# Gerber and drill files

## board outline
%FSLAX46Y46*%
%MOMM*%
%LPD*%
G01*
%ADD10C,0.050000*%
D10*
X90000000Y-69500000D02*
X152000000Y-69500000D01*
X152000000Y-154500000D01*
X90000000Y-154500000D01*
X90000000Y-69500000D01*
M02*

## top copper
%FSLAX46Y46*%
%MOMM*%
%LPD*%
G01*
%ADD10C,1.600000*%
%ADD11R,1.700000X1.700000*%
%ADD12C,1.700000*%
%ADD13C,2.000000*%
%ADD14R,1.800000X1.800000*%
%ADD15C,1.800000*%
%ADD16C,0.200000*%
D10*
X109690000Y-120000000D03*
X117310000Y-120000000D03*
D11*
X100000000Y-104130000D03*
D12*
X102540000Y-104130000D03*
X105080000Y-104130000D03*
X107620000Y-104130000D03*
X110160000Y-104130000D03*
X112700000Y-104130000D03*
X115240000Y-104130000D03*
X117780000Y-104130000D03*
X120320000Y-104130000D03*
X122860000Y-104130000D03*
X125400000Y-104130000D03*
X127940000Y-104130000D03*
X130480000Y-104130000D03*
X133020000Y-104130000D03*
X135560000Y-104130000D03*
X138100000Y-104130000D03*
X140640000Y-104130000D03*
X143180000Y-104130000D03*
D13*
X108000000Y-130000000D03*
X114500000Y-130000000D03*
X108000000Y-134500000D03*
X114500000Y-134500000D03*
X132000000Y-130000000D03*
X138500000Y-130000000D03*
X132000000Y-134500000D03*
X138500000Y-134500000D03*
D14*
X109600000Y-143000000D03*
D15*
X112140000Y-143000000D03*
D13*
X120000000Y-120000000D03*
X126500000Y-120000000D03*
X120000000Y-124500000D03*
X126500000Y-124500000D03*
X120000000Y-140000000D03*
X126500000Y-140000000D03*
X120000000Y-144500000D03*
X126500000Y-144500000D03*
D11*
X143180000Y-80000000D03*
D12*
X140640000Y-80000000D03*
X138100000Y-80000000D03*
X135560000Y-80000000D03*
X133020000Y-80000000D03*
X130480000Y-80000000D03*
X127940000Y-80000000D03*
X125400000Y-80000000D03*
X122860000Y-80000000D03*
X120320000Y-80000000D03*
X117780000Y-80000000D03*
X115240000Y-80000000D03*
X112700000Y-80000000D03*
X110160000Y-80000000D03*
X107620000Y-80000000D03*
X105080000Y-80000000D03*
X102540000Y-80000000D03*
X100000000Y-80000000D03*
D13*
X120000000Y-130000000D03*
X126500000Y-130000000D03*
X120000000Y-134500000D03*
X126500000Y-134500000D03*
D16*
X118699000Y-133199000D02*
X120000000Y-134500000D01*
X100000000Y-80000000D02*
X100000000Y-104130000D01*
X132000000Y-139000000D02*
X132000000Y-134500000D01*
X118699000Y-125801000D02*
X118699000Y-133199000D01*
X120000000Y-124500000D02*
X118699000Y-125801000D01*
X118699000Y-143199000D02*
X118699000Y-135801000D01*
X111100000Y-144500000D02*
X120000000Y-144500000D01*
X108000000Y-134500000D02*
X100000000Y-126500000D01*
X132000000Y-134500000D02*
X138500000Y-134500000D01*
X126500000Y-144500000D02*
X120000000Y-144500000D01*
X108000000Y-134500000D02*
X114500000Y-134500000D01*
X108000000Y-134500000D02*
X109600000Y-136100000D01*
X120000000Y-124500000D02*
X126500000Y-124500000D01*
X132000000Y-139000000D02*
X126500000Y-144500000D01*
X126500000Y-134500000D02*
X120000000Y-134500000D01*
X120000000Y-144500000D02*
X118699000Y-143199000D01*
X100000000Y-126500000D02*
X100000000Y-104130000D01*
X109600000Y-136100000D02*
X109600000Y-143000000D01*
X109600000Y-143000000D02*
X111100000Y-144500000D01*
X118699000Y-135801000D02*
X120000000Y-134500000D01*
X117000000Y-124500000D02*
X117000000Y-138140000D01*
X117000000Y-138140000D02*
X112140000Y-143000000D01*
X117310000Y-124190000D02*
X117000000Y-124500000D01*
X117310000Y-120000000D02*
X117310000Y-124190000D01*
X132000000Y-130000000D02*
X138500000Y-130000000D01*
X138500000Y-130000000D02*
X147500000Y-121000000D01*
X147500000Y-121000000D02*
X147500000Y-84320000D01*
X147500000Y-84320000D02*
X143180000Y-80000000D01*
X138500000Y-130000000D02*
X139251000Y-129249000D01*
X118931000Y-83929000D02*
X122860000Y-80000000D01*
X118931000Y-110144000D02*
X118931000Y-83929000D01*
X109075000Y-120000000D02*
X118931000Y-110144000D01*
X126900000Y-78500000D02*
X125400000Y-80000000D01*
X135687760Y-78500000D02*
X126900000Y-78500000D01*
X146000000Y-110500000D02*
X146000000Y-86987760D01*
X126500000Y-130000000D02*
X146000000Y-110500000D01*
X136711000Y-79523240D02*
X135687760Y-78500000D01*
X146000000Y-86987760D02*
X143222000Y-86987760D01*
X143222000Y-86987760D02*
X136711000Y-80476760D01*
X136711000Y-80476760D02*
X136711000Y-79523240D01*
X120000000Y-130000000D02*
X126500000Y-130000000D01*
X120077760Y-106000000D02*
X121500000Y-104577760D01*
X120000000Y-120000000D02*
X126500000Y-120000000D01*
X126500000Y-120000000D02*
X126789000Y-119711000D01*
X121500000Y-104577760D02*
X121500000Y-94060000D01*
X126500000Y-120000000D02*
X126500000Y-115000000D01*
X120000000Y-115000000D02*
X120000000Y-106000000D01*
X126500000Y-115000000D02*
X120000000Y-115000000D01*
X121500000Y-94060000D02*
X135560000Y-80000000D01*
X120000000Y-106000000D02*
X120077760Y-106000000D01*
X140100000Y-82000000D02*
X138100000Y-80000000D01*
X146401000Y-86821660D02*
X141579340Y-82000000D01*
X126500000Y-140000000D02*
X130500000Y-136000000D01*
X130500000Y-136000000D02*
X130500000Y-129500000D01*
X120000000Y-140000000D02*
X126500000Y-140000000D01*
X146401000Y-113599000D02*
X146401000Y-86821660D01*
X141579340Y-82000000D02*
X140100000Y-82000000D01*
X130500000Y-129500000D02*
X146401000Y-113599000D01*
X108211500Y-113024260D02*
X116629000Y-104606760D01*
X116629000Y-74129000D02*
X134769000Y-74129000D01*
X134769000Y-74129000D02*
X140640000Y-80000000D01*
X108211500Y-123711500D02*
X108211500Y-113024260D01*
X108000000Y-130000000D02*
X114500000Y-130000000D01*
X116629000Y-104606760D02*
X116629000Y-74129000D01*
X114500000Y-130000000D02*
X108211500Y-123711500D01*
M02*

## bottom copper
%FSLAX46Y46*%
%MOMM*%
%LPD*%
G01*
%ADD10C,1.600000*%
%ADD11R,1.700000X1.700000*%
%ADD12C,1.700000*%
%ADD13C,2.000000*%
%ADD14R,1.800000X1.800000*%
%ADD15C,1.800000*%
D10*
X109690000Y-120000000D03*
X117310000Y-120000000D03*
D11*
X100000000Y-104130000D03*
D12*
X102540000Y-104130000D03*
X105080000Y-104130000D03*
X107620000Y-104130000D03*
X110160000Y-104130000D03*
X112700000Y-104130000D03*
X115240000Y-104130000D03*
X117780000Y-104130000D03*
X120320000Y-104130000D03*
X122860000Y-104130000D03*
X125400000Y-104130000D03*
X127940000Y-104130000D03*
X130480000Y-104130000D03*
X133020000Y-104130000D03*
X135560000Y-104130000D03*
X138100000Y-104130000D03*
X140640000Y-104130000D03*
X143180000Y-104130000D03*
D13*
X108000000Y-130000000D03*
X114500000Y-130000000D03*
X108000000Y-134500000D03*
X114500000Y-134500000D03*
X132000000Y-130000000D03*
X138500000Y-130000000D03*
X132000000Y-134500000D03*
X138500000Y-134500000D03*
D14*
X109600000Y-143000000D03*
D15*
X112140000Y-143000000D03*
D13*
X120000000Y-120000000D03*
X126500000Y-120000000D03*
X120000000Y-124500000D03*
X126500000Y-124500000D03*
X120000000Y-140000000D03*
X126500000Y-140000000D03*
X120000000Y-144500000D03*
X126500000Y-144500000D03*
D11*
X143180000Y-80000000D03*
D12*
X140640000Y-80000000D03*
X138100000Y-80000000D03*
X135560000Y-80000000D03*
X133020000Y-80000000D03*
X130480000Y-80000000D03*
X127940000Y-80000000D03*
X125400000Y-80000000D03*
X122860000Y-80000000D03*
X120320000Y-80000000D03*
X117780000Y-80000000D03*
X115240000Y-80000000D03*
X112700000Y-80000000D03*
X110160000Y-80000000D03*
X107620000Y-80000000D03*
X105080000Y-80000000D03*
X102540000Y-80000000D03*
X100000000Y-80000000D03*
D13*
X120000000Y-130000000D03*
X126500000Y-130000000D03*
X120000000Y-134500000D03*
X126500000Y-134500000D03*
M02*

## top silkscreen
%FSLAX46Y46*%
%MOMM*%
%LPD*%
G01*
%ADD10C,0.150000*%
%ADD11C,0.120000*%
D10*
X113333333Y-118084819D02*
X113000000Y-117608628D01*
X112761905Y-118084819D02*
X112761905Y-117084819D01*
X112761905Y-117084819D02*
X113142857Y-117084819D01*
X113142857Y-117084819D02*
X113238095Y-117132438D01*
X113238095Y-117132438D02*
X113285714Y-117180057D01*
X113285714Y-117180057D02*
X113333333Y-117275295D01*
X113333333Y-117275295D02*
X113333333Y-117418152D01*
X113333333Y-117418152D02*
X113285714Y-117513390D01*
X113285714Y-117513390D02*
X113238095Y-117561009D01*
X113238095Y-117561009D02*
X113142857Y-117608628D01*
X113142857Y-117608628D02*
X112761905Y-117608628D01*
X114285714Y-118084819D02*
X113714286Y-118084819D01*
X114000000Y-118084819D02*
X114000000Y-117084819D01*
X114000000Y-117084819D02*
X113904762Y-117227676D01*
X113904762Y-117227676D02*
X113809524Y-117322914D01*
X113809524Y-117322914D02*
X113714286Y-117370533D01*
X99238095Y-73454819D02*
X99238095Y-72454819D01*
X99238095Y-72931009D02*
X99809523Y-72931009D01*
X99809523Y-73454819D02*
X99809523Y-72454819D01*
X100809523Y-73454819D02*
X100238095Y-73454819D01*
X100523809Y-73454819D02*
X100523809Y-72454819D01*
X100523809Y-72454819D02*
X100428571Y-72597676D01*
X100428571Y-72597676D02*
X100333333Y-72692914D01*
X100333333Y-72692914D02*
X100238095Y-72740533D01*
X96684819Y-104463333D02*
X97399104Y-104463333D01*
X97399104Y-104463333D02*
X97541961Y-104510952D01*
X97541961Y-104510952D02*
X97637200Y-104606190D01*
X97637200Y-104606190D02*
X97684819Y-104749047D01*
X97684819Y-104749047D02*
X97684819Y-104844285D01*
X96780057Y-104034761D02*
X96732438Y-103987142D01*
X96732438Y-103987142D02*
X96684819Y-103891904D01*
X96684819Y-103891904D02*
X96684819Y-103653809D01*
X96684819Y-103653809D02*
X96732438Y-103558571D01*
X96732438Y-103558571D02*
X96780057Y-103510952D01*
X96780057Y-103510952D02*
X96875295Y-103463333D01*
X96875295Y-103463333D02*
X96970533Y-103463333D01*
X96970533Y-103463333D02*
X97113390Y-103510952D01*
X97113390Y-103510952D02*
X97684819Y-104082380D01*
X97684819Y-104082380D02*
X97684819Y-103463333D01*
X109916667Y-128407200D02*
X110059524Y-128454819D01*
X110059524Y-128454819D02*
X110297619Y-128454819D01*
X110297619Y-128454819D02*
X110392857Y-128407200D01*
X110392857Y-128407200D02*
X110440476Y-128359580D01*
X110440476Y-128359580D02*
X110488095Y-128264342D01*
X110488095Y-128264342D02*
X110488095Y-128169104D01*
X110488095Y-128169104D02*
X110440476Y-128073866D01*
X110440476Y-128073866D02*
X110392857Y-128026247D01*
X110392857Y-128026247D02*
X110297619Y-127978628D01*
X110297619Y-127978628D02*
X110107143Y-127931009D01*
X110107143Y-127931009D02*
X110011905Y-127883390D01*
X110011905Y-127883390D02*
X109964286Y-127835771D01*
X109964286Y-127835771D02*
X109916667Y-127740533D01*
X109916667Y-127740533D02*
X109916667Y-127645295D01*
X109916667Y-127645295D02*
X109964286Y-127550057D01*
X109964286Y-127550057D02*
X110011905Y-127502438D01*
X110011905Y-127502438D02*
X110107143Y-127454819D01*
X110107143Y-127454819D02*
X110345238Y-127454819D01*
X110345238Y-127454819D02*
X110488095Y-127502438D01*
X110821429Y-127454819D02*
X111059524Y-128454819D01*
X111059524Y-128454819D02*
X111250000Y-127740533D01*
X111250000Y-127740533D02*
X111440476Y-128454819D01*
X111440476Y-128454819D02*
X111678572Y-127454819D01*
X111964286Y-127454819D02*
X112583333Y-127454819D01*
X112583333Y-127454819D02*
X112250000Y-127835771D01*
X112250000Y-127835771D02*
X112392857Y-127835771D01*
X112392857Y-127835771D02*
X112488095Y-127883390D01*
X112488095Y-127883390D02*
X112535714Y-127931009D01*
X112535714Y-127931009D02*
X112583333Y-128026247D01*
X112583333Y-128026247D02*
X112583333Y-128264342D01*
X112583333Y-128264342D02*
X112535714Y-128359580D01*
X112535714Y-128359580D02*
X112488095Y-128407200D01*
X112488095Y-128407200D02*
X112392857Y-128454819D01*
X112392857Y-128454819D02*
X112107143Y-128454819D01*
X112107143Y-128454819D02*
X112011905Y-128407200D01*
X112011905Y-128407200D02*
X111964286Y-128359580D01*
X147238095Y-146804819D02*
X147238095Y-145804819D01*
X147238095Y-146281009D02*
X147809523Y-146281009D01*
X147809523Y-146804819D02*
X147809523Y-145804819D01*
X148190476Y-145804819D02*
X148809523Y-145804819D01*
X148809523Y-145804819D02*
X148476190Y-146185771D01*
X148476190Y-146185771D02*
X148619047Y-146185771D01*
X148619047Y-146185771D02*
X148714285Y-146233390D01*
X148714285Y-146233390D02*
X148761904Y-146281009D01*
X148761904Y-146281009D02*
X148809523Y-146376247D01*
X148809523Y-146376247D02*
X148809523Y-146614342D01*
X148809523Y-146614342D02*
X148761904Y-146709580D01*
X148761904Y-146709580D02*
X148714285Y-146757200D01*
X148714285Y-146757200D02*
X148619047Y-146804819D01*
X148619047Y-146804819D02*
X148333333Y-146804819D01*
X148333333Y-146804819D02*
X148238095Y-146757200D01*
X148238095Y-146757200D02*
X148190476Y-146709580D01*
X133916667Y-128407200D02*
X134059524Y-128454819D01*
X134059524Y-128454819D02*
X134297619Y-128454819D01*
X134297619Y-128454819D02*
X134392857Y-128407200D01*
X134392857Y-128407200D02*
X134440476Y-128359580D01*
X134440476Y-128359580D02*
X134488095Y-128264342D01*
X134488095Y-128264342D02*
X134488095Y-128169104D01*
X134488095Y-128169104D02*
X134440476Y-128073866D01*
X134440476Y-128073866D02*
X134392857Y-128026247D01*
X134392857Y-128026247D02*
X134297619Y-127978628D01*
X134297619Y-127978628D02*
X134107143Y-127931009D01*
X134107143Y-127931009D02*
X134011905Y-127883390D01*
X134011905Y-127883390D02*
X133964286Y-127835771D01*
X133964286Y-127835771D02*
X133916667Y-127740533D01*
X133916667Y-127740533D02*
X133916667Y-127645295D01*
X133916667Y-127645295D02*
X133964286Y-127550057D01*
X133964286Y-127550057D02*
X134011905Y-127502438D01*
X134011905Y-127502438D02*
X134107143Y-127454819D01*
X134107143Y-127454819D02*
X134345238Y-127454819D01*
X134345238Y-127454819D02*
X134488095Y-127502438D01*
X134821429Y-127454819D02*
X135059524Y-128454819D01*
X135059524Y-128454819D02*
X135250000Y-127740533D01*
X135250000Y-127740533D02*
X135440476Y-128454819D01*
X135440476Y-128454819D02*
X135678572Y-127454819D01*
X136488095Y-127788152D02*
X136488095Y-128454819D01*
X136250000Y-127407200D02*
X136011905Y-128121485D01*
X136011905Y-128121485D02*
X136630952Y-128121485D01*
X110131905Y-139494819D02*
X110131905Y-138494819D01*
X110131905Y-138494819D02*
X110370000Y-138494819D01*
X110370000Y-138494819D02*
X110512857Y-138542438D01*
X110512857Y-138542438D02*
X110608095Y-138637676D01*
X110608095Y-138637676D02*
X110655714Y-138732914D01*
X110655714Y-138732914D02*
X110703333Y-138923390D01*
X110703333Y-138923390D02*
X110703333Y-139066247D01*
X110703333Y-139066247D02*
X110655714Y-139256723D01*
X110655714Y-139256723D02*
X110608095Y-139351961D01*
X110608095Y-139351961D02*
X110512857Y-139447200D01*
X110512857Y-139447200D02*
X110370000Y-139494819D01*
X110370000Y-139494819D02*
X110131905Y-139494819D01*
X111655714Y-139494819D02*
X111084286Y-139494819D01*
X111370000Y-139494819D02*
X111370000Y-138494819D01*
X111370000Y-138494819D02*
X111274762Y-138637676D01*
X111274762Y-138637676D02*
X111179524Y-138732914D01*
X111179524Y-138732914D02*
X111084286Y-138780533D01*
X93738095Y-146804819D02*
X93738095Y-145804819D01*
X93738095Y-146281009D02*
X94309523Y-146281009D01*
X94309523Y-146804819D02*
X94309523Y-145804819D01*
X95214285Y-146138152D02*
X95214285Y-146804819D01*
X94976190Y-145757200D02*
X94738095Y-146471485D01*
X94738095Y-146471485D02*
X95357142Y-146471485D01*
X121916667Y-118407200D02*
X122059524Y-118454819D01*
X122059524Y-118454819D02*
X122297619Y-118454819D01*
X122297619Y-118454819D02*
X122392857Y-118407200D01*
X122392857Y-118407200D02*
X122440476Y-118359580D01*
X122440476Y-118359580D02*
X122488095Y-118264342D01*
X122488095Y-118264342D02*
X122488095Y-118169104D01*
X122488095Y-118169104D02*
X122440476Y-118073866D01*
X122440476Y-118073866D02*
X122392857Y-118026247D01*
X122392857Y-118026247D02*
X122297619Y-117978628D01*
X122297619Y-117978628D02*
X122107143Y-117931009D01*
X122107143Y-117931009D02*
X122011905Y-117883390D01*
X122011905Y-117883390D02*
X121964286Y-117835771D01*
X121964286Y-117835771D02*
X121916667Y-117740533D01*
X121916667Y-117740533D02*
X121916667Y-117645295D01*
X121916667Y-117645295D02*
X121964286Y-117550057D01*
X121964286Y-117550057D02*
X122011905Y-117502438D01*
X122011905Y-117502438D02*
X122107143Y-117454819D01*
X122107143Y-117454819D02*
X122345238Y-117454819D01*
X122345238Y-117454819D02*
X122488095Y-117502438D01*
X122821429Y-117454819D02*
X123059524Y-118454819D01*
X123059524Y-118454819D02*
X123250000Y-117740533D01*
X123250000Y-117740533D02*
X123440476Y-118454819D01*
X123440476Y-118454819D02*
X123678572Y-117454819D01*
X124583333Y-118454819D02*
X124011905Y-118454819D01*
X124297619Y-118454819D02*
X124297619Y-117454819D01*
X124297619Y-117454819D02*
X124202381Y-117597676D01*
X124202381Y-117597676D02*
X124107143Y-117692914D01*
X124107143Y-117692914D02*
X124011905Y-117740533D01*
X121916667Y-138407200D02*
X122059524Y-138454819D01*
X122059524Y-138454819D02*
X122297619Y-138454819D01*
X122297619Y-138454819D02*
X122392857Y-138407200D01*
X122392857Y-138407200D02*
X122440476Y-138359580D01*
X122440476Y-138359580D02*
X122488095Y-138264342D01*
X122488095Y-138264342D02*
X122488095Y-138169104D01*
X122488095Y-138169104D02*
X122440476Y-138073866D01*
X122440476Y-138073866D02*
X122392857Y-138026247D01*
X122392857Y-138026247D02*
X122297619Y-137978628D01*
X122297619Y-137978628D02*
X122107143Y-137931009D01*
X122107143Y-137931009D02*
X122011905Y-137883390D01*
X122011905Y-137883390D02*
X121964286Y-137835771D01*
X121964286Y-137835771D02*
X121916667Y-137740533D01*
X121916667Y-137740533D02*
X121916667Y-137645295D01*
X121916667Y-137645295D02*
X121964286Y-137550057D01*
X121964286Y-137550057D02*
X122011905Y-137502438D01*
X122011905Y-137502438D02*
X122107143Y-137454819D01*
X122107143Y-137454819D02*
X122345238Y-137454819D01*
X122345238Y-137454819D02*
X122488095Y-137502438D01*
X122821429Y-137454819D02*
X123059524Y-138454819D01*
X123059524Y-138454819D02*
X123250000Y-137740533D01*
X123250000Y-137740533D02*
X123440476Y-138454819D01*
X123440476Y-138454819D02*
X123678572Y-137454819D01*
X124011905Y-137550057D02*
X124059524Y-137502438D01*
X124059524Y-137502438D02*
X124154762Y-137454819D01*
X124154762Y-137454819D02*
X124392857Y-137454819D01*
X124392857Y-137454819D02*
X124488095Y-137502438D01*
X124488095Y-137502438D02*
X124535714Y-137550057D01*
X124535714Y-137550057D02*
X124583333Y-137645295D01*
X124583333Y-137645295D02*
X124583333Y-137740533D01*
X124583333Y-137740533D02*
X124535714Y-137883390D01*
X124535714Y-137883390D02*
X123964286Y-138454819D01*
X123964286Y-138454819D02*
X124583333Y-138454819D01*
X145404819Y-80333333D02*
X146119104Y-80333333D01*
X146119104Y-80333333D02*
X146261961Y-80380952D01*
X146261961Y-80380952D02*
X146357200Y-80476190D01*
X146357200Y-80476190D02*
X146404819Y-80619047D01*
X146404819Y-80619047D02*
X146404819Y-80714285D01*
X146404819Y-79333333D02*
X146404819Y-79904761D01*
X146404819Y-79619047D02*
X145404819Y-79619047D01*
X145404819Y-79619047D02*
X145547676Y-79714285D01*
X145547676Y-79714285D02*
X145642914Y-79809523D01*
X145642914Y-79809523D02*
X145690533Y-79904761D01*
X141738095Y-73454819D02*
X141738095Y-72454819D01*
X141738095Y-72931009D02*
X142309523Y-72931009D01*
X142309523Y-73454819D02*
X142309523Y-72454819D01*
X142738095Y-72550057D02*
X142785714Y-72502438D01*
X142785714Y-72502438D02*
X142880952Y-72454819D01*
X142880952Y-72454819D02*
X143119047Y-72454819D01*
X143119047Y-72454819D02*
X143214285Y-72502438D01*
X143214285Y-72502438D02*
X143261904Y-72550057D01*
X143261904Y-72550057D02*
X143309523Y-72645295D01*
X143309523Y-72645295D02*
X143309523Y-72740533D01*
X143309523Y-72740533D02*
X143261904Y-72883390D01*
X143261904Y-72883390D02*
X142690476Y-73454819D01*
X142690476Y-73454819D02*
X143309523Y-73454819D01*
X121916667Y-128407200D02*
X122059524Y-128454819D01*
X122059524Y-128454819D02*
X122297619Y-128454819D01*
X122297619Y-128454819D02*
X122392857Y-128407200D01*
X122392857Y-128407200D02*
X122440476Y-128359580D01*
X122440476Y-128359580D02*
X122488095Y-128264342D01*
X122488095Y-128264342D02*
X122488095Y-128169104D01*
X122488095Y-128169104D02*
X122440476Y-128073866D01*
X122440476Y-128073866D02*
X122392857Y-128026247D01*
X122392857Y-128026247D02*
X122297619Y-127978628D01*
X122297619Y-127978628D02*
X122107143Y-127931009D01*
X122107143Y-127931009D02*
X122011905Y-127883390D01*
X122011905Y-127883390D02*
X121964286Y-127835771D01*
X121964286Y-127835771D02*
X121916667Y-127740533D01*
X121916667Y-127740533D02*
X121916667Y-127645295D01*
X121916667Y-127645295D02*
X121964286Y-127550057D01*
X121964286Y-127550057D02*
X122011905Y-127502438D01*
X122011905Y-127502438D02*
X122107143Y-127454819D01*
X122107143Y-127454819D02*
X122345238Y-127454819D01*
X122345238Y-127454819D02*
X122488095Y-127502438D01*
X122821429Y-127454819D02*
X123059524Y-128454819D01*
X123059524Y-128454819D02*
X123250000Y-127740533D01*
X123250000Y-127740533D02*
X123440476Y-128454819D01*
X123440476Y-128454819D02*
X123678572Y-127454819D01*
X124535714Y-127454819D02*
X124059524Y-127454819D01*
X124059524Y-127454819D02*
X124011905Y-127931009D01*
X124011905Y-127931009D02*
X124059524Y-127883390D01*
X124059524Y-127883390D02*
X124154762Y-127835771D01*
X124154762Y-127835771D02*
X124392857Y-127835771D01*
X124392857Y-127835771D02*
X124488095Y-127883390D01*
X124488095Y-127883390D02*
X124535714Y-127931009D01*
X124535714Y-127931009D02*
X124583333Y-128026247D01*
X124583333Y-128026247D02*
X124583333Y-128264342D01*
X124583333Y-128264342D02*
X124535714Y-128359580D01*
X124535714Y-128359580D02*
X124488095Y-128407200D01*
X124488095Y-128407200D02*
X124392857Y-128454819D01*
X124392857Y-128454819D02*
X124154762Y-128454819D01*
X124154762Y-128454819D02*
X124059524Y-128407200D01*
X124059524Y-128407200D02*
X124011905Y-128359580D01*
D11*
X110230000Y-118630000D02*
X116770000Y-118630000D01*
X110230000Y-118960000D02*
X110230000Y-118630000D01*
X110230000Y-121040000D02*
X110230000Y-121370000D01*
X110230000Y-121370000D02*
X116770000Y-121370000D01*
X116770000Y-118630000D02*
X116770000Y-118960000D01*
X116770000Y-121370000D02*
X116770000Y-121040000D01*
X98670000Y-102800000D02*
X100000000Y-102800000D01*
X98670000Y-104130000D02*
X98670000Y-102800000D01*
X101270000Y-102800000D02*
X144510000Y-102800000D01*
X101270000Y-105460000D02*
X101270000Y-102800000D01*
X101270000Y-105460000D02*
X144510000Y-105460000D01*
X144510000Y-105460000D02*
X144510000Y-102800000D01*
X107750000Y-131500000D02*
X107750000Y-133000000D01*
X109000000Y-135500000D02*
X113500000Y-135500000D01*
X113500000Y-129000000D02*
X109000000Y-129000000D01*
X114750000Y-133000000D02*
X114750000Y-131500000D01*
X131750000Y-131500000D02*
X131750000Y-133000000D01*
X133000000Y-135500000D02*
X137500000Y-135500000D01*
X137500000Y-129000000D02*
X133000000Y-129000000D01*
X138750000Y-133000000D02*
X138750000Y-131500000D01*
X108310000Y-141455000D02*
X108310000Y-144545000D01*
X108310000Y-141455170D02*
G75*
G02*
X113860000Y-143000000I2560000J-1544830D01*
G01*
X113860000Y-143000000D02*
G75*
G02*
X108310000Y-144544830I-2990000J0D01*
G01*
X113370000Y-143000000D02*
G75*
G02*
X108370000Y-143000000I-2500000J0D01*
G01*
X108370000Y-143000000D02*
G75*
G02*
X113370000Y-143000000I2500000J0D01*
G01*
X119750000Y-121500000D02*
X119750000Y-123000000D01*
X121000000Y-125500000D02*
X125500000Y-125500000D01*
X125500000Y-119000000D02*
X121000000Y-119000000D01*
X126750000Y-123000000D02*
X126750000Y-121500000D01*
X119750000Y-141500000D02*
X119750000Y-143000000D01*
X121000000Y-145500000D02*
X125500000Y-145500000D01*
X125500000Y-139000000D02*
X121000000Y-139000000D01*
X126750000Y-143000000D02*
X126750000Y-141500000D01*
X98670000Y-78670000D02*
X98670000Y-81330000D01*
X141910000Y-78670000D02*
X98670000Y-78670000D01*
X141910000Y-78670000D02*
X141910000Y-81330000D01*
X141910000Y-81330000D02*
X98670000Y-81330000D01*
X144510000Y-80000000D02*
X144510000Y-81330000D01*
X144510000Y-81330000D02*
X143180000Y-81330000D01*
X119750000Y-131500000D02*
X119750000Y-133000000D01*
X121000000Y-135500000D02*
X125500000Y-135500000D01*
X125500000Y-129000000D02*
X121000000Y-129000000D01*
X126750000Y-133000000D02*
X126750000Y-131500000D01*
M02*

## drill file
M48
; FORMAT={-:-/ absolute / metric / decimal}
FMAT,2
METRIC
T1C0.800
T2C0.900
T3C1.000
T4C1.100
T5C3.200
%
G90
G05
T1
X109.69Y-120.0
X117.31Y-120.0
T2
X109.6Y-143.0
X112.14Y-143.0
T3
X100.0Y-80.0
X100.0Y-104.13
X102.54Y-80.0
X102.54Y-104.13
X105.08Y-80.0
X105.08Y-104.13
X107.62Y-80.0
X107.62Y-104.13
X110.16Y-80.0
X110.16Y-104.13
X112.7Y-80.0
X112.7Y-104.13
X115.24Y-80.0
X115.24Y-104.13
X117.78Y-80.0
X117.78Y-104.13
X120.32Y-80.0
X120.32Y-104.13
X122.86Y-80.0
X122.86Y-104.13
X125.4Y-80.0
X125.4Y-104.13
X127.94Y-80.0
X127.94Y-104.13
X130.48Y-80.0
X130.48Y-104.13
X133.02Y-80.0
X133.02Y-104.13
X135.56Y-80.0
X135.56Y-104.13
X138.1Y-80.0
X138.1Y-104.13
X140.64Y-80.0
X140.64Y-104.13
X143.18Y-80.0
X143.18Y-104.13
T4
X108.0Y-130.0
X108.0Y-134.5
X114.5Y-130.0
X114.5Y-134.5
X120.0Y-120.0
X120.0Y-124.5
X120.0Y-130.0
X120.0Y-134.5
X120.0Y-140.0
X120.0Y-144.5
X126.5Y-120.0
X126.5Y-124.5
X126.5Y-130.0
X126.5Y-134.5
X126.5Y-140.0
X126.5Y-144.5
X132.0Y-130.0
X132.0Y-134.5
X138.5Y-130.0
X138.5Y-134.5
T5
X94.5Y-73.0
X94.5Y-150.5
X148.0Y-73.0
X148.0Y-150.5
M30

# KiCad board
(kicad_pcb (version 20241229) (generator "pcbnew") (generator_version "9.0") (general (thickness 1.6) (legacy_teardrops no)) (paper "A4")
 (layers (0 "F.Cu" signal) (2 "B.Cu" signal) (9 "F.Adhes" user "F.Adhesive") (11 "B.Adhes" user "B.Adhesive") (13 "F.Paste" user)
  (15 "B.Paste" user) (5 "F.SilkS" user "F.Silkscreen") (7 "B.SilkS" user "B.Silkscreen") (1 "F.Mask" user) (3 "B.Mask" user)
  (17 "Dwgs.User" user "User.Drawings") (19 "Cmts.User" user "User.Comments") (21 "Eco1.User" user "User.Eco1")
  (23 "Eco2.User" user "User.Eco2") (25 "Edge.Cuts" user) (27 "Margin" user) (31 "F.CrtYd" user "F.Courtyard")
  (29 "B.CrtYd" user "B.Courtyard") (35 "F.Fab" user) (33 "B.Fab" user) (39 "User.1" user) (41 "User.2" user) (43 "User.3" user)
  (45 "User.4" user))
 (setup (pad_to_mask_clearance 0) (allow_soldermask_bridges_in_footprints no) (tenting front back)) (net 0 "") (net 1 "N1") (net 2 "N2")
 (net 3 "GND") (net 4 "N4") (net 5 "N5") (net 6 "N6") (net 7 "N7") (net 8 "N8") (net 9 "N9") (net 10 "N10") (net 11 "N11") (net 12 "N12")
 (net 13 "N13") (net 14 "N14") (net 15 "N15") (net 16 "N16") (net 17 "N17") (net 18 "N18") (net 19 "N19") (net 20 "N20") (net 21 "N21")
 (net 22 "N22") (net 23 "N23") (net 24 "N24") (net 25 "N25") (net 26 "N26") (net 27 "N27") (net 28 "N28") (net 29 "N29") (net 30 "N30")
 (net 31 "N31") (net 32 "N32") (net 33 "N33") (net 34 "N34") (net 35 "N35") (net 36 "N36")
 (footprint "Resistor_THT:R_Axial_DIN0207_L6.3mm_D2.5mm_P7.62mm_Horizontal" (layer "F.Cu") (at 109.69 120)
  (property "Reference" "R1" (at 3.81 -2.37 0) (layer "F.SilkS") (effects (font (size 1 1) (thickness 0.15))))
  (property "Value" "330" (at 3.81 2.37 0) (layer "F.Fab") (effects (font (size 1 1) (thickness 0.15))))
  (fp_line (start 0.54 -1.37) (end 7.08 -1.37) (stroke (width 0.12) (type solid)) (layer "F.SilkS"))
  (fp_line (start 0.54 -1.04) (end 0.54 -1.37) (stroke (width 0.12) (type solid)) (layer "F.SilkS"))
  (fp_line (start 0.54 1.04) (end 0.54 1.37) (stroke (width 0.12) (type solid)) (layer "F.SilkS"))
  (fp_line (start 0.54 1.37) (end 7.08 1.37) (stroke (width 0.12) (type solid)) (layer "F.SilkS"))
  (fp_line (start 7.08 -1.37) (end 7.08 -1.04) (stroke (width 0.12) (type solid)) (layer "F.SilkS"))
  (fp_line (start 7.08 1.37) (end 7.08 1.04) (stroke (width 0.12) (type solid)) (layer "F.SilkS"))
  (pad "1" thru_hole circle (at 0 0) (size 1.6 1.6) (drill 0.8) (layers "*.Cu" "*.Mask") (remove_unused_layers no) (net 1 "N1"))
  (pad "2" thru_hole circle (at 7.62 0) (size 1.6 1.6) (drill 0.8) (layers "*.Cu" "*.Mask") (remove_unused_layers no) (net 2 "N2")))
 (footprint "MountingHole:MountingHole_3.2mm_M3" (layer "F.Cu") (at 94.5 73)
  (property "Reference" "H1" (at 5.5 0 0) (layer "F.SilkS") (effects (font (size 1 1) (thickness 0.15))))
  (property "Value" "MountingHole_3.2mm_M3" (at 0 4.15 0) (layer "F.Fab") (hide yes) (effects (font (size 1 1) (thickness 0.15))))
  (pad "" np_thru_hole circle (at 0 0) (size 3.2 3.2) (drill 3.2) (layers "*.Cu" "*.Mask")))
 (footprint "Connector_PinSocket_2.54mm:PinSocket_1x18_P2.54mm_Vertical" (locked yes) (layer "F.Cu") (at 100 104.13 90)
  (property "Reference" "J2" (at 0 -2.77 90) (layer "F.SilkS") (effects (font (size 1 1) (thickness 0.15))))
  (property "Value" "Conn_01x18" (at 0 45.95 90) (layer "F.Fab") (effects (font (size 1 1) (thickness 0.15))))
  (fp_line (start 1.33 -1.33) (end 1.33 0) (stroke (width 0.12) (type solid)) (layer "F.SilkS"))
  (fp_line (start 0 -1.33) (end 1.33 -1.33) (stroke (width 0.12) (type solid)) (layer "F.SilkS"))
  (fp_line (start 1.33 1.27) (end 1.33 44.51) (stroke (width 0.12) (type solid)) (layer "F.SilkS"))
  (fp_line (start -1.33 1.27) (end 1.33 1.27) (stroke (width 0.12) (type solid)) (layer "F.SilkS"))
  (fp_line (start -1.33 1.27) (end -1.33 44.51) (stroke (width 0.12) (type solid)) (layer "F.SilkS"))
  (fp_line (start -1.33 44.51) (end 1.33 44.51) (stroke (width 0.12) (type solid)) (layer "F.SilkS"))
  (pad "1" thru_hole rect (at 0 0 90) (size 1.7 1.7) (drill 1) (layers "*.Cu" "*.Mask") (remove_unused_layers no) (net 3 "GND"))
  (pad "2" thru_hole circle (at 0 2.54 90) (size 1.7 1.7) (drill 1) (layers "*.Cu" "*.Mask") (remove_unused_layers no) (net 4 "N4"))
  (pad "3" thru_hole circle (at 0 5.08 90) (size 1.7 1.7) (drill 1) (layers "*.Cu" "*.Mask") (remove_unused_layers no) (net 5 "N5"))
  (pad "4" thru_hole circle (at 0 7.62 90) (size 1.7 1.7) (drill 1) (layers "*.Cu" "*.Mask") (remove_unused_layers no) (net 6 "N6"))
  (pad "5" thru_hole circle (at 0 10.16 90) (size 1.7 1.7) (drill 1) (layers "*.Cu" "*.Mask") (remove_unused_layers no) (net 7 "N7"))
  (pad "6" thru_hole circle (at 0 12.7 90) (size 1.7 1.7) (drill 1) (layers "*.Cu" "*.Mask") (remove_unused_layers no) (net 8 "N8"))
  (pad "7" thru_hole circle (at 0 15.24 90) (size 1.7 1.7) (drill 1) (layers "*.Cu" "*.Mask") (remove_unused_layers no) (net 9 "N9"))
  (pad "8" thru_hole circle (at 0 17.78 90) (size 1.7 1.7) (drill 1) (layers "*.Cu" "*.Mask") (remove_unused_layers no) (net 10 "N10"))
  (pad "9" thru_hole circle (at 0 20.32 90) (size 1.7 1.7) (drill 1) (layers "*.Cu" "*.Mask") (remove_unused_layers no) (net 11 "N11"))
  (pad "10" thru_hole circle (at 0 22.86 90) (size 1.7 1.7) (drill 1) (layers "*.Cu" "*.Mask") (remove_unused_layers no) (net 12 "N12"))
  (pad "11" thru_hole circle (at 0 25.4 90) (size 1.7 1.7) (drill 1) (layers "*.Cu" "*.Mask") (remove_unused_layers no) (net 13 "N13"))
  (pad "12" thru_hole circle (at 0 27.94 90) (size 1.7 1.7) (drill 1) (layers "*.Cu" "*.Mask") (remove_unused_layers no) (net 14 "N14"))
  (pad "13" thru_hole circle (at 0 30.48 90) (size 1.7 1.7) (drill 1) (layers "*.Cu" "*.Mask") (remove_unused_layers no) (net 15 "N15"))
  (pad "14" thru_hole circle (at 0 33.02 90) (size 1.7 1.7) (drill 1) (layers "*.Cu" "*.Mask") (remove_unused_layers no) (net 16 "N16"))
  (pad "15" thru_hole circle (at 0 35.56 90) (size 1.7 1.7) (drill 1) (layers "*.Cu" "*.Mask") (remove_unused_layers no) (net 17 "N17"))
  (pad "16" thru_hole circle (at 0 38.1 90) (size 1.7 1.7) (drill 1) (layers "*.Cu" "*.Mask") (remove_unused_layers no) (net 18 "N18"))
  (pad "17" thru_hole circle (at 0 40.64 90) (size 1.7 1.7) (drill 1) (layers "*.Cu" "*.Mask") (remove_unused_layers no) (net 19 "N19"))
  (pad "18" thru_hole circle (at 0 43.18 90) (size 1.7 1.7) (drill 1) (layers "*.Cu" "*.Mask") (remove_unused_layers no) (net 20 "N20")))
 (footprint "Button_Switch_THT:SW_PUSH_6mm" (layer "F.Cu") (at 108 130)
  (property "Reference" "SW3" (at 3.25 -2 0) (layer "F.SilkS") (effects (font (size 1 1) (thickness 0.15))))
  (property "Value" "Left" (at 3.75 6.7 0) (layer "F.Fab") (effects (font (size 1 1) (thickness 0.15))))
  (fp_line (start -0.25 1.5) (end -0.25 3) (stroke (width 0.12) (type solid)) (layer "F.SilkS"))
  (fp_line (start 1 5.5) (end 5.5 5.5) (stroke (width 0.12) (type solid)) (layer "F.SilkS"))
  (fp_line (start 5.5 -1) (end 1 -1) (stroke (width 0.12) (type solid)) (layer "F.SilkS"))
  (fp_line (start 6.75 3) (end 6.75 1.5) (stroke (width 0.12) (type solid)) (layer "F.SilkS"))
  (pad "1" thru_hole circle (at 0 0 90) (size 2 2) (drill 1.1) (layers "*.Cu" "*.Mask") (remove_unused_layers no) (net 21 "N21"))
  (pad "1" thru_hole circle (at 6.5 0 90) (size 2 2) (drill 1.1) (layers "*.Cu" "*.Mask") (remove_unused_layers no) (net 21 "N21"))
  (pad "2" thru_hole circle (at 0 4.5 90) (size 2 2) (drill 1.1) (layers "*.Cu" "*.Mask") (remove_unused_layers no) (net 3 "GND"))
  (pad "2" thru_hole circle (at 6.5 4.5 90) (size 2 2) (drill 1.1) (layers "*.Cu" "*.Mask") (remove_unused_layers no) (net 3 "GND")))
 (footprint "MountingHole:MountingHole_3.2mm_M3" (layer "F.Cu") (at 148 150.5)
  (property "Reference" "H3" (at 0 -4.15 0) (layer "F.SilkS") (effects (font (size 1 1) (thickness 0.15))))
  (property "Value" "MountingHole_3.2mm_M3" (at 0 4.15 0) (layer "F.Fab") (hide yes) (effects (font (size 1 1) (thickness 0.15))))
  (pad "" np_thru_hole circle (at 0 0) (size 3.2 3.2) (drill 3.2) (layers "*.Cu" "*.Mask")))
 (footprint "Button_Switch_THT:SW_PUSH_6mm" (layer "F.Cu") (at 132 130)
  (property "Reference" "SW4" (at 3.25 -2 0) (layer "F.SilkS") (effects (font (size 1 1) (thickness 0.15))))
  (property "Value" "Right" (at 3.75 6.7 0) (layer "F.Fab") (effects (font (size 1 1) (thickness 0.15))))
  (fp_line (start -0.25 1.5) (end -0.25 3) (stroke (width 0.12) (type solid)) (layer "F.SilkS"))
  (fp_line (start 1 5.5) (end 5.5 5.5) (stroke (width 0.12) (type solid)) (layer "F.SilkS"))
  (fp_line (start 5.5 -1) (end 1 -1) (stroke (width 0.12) (type solid)) (layer "F.SilkS"))
  (fp_line (start 6.75 3) (end 6.75 1.5) (stroke (width 0.12) (type solid)) (layer "F.SilkS"))
  (pad "1" thru_hole circle (at 0 0 90) (size 2 2) (drill 1.1) (layers "*.Cu" "*.Mask") (remove_unused_layers no) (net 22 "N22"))
  (pad "1" thru_hole circle (at 6.5 0 90) (size 2 2) (drill 1.1) (layers "*.Cu" "*.Mask") (remove_unused_layers no) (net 22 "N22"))
  (pad "2" thru_hole circle (at 0 4.5 90) (size 2 2) (drill 1.1) (layers "*.Cu" "*.Mask") (remove_unused_layers no) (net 3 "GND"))
  (pad "2" thru_hole circle (at 6.5 4.5 90) (size 2 2) (drill 1.1) (layers "*.Cu" "*.Mask") (remove_unused_layers no) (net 3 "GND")))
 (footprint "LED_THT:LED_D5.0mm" (layer "F.Cu") (at 109.6 143)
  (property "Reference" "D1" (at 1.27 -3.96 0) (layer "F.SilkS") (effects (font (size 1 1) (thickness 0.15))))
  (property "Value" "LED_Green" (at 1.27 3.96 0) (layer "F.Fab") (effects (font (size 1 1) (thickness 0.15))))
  (fp_line (start -1.29 -1.545) (end -1.29 1.545) (stroke (width 0.12) (type solid)) (layer "F.SilkS"))
  (fp_arc (start -1.29 -1.54483) (mid 2.071779 -2.880495) (end 4.26 0) (stroke (width 0.12) (type solid)) (layer "F.SilkS"))
  (fp_arc (start 4.26 0) (mid 2.071779 2.880495) (end -1.29 1.54483) (stroke (width 0.12) (type solid)) (layer "F.SilkS"))
  (fp_circle (center 1.27 0) (end 3.77 0) (stroke (width 0.12) (type solid)) (fill no) (layer "F.SilkS"))
  (pad "1" thru_hole rect (at 0 0) (size 1.8 1.8) (drill 0.9) (layers "*.Cu" "*.Mask") (remove_unused_layers no) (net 3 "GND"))
  (pad "2" thru_hole circle (at 2.54 0) (size 1.8 1.8) (drill 0.9) (layers "*.Cu" "*.Mask") (remove_unused_layers no) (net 2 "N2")))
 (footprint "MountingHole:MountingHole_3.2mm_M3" (layer "F.Cu") (at 94.5 150.5)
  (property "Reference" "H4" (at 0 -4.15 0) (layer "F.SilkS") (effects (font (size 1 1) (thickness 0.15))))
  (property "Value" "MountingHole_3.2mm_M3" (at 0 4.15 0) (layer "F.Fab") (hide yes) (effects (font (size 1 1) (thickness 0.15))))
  (pad "" np_thru_hole circle (at 0 0) (size 3.2 3.2) (drill 3.2) (layers "*.Cu" "*.Mask")))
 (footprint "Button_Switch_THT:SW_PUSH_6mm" (layer "F.Cu") (at 120 120)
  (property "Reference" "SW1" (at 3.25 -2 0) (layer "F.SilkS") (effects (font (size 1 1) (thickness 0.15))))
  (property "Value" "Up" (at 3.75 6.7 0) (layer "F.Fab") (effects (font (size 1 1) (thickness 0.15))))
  (fp_line (start -0.25 1.5) (end -0.25 3) (stroke (width 0.12) (type solid)) (layer "F.SilkS"))
  (fp_line (start 1 5.5) (end 5.5 5.5) (stroke (width 0.12) (type solid)) (layer "F.SilkS"))
  (fp_line (start 5.5 -1) (end 1 -1) (stroke (width 0.12) (type solid)) (layer "F.SilkS"))
  (fp_line (start 6.75 3) (end 6.75 1.5) (stroke (width 0.12) (type solid)) (layer "F.SilkS"))
  (pad "1" thru_hole circle (at 0 0 90) (size 2 2) (drill 1.1) (layers "*.Cu" "*.Mask") (remove_unused_layers no) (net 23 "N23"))
  (pad "1" thru_hole circle (at 6.5 0 90) (size 2 2) (drill 1.1) (layers "*.Cu" "*.Mask") (remove_unused_layers no) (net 23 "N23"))
  (pad "2" thru_hole circle (at 0 4.5 90) (size 2 2) (drill 1.1) (layers "*.Cu" "*.Mask") (remove_unused_layers no) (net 3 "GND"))
  (pad "2" thru_hole circle (at 6.5 4.5 90) (size 2 2) (drill 1.1) (layers "*.Cu" "*.Mask") (remove_unused_layers no) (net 3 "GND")))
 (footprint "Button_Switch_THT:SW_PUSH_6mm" (layer "F.Cu") (at 120 140)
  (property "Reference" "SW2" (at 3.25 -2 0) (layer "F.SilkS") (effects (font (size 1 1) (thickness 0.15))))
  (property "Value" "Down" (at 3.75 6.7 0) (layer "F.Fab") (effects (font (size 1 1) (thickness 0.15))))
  (fp_line (start -0.25 1.5) (end -0.25 3) (stroke (width 0.12) (type solid)) (layer "F.SilkS"))
  (fp_line (start 1 5.5) (end 5.5 5.5) (stroke (width 0.12) (type solid)) (layer "F.SilkS"))
  (fp_line (start 5.5 -1) (end 1 -1) (stroke (width 0.12) (type solid)) (layer "F.SilkS"))
  (fp_line (start 6.75 3) (end 6.75 1.5) (stroke (width 0.12) (type solid)) (layer "F.SilkS"))
  (pad "1" thru_hole circle (at 0 0 90) (size 2 2) (drill 1.1) (layers "*.Cu" "*.Mask") (remove_unused_layers no) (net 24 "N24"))
  (pad "1" thru_hole circle (at 6.5 0 90) (size 2 2) (drill 1.1) (layers "*.Cu" "*.Mask") (remove_unused_layers no) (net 24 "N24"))
  (pad "2" thru_hole circle (at 0 4.5 90) (size 2 2) (drill 1.1) (layers "*.Cu" "*.Mask") (remove_unused_layers no) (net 3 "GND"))
  (pad "2" thru_hole circle (at 6.5 4.5 90) (size 2 2) (drill 1.1) (layers "*.Cu" "*.Mask") (remove_unused_layers no) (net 3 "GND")))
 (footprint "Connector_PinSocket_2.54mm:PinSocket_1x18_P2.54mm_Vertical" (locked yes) (layer "F.Cu") (at 143.18 80 -90)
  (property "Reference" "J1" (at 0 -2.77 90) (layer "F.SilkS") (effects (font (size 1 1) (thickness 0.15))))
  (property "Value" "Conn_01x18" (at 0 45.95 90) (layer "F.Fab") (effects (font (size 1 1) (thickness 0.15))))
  (fp_line (start -1.33 44.51) (end 1.33 44.51) (stroke (width 0.12) (type solid)) (layer "F.SilkS"))
  (fp_line (start -1.33 1.27) (end -1.33 44.51) (stroke (width 0.12) (type solid)) (layer "F.SilkS"))
  (fp_line (start -1.33 1.27) (end 1.33 1.27) (stroke (width 0.12) (type solid)) (layer "F.SilkS"))
  (fp_line (start 1.33 1.27) (end 1.33 44.51) (stroke (width 0.12) (type solid)) (layer "F.SilkS"))
  (fp_line (start 0 -1.33) (end 1.33 -1.33) (stroke (width 0.12) (type solid)) (layer "F.SilkS"))
  (fp_line (start 1.33 -1.33) (end 1.33 0) (stroke (width 0.12) (type solid)) (layer "F.SilkS"))
  (pad "1" thru_hole rect (at 0 0 270) (size 1.7 1.7) (drill 1) (layers "*.Cu" "*.Mask") (remove_unused_layers no) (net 22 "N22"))
  (pad "2" thru_hole circle (at 0 2.54 270) (size 1.7 1.7) (drill 1) (layers "*.Cu" "*.Mask") (remove_unused_layers no) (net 21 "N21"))
  (pad "3" thru_hole circle (at 0 5.08 270) (size 1.7 1.7) (drill 1) (layers "*.Cu" "*.Mask") (remove_unused_layers no) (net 24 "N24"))
  (pad "4" thru_hole circle (at 0 7.62 270) (size 1.7 1.7) (drill 1) (layers "*.Cu" "*.Mask") (remove_unused_layers no) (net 23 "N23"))
  (pad "5" thru_hole circle (at 0 10.16 270) (size 1.7 1.7) (drill 1) (layers "*.Cu" "*.Mask") (remove_unused_layers no) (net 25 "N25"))
  (pad "6" thru_hole circle (at 0 12.7 270) (size 1.7 1.7) (drill 1) (layers "*.Cu" "*.Mask") (remove_unused_layers no) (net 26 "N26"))
  (pad "7" thru_hole circle (at 0 15.24 270) (size 1.7 1.7) (drill 1) (layers "*.Cu" "*.Mask") (remove_unused_layers no) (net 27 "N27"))
  (pad "8" thru_hole circle (at 0 17.78 270) (size 1.7 1.7) (drill 1) (layers "*.Cu" "*.Mask") (remove_unused_layers no) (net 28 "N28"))
  (pad "9" thru_hole circle (at 0 20.32 270) (size 1.7 1.7) (drill 1) (layers "*.Cu" "*.Mask") (remove_unused_layers no) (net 1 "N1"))
  (pad "10" thru_hole circle (at 0 22.86 270) (size 1.7 1.7) (drill 1) (layers "*.Cu" "*.Mask") (remove_unused_layers no) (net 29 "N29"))
  (pad "11" thru_hole circle (at 0 25.4 270) (size 1.7 1.7) (drill 1) (layers "*.Cu" "*.Mask") (remove_unused_layers no) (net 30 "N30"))
  (pad "12" thru_hole circle (at 0 27.94 270) (size 1.7 1.7) (drill 1) (layers "*.Cu" "*.Mask") (remove_unused_layers no) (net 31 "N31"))
  (pad "13" thru_hole circle (at 0 30.48 270) (size 1.7 1.7) (drill 1) (layers "*.Cu" "*.Mask") (remove_unused_layers no) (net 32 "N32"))
  (pad "14" thru_hole circle (at 0 33.02 270) (size 1.7 1.7) (drill 1) (layers "*.Cu" "*.Mask") (remove_unused_layers no) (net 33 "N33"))
  (pad "15" thru_hole circle (at 0 35.56 270) (size 1.7 1.7) (drill 1) (layers "*.Cu" "*.Mask") (remove_unused_layers no) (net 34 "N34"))
  (pad "16" thru_hole circle (at 0 38.1 270) (size 1.7 1.7) (drill 1) (layers "*.Cu" "*.Mask") (remove_unused_layers no) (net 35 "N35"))
  (pad "17" thru_hole circle (at 0 40.64 270) (size 1.7 1.7) (drill 1) (layers "*.Cu" "*.Mask") (remove_unused_layers no) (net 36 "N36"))
  (pad "18" thru_hole circle (at 0 43.18 270) (size 1.7 1.7) (drill 1) (layers "*.Cu" "*.Mask") (remove_unused_layers no) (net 3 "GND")))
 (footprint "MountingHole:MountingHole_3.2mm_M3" (layer "F.Cu") (at 148 73)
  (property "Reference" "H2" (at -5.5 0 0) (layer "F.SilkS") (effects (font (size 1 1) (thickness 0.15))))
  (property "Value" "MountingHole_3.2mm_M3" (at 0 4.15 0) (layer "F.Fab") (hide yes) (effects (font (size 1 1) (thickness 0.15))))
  (pad "" np_thru_hole circle (at 0 0) (size 3.2 3.2) (drill 3.2) (layers "*.Cu" "*.Mask")))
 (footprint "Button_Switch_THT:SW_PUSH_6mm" (layer "F.Cu") (at 120 130)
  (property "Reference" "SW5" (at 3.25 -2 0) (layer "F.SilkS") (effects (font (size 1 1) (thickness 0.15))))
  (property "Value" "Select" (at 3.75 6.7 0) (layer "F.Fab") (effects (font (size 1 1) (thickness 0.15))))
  (fp_line (start -0.25 1.5) (end -0.25 3) (stroke (width 0.12) (type solid)) (layer "F.SilkS"))
  (fp_line (start 1 5.5) (end 5.5 5.5) (stroke (width 0.12) (type solid)) (layer "F.SilkS"))
  (fp_line (start 5.5 -1) (end 1 -1) (stroke (width 0.12) (type solid)) (layer "F.SilkS"))
  (fp_line (start 6.75 3) (end 6.75 1.5) (stroke (width 0.12) (type solid)) (layer "F.SilkS"))
  (pad "1" thru_hole circle (at 0 0 90) (size 2 2) (drill 1.1) (layers "*.Cu" "*.Mask") (remove_unused_layers no) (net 28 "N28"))
  (pad "1" thru_hole circle (at 6.5 0 90) (size 2 2) (drill 1.1) (layers "*.Cu" "*.Mask") (remove_unused_layers no) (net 28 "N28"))
  (pad "2" thru_hole circle (at 0 4.5 90) (size 2 2) (drill 1.1) (layers "*.Cu" "*.Mask") (remove_unused_layers no) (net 3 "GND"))
  (pad "2" thru_hole circle (at 6.5 4.5 90) (size 2 2) (drill 1.1) (layers "*.Cu" "*.Mask") (remove_unused_layers no) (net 3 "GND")))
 (gr_rect (start 90 69.5) (end 152 154.5) (stroke (width 0.05) (type default)) (fill no) (layer "Edge.Cuts"))
 (segment (start 118.699 133.199) (end 120 134.5) (width 0.2) (layer "F.Cu") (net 3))
 (segment (start 100 80) (end 100 104.13) (width 0.2) (layer "F.Cu") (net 3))
 (segment (start 132 139) (end 132 134.5) (width 0.2) (layer "F.Cu") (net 3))
 (segment (start 118.699 125.801) (end 118.699 133.199) (width 0.2) (layer "F.Cu") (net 3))
 (segment (start 120 124.5) (end 118.699 125.801) (width 0.2) (layer "F.Cu") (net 3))
 (segment (start 118.699 143.199) (end 118.699 135.801) (width 0.2) (layer "F.Cu") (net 3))
 (segment (start 111.1 144.5) (end 120 144.5) (width 0.2) (layer "F.Cu") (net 3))
 (segment (start 108 134.5) (end 100 126.5) (width 0.2) (layer "F.Cu") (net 3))
 (segment (start 132 134.5) (end 138.5 134.5) (width 0.2) (layer "F.Cu") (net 3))
 (segment (start 126.5 144.5) (end 120 144.5) (width 0.2) (layer "F.Cu") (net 3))
 (segment (start 108 134.5) (end 114.5 134.5) (width 0.2) (layer "F.Cu") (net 3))
 (segment (start 108 134.5) (end 109.6 136.1) (width 0.2) (layer "F.Cu") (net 3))
 (segment (start 120 124.5) (end 126.5 124.5) (width 0.2) (layer "F.Cu") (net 3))
 (segment (start 132 139) (end 126.5 144.5) (width 0.2) (layer "F.Cu") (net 3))
 (segment (start 126.5 134.5) (end 120 134.5) (width 0.2) (layer "F.Cu") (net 3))
 (segment (start 120 144.5) (end 118.699 143.199) (width 0.2) (layer "F.Cu") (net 3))
 (segment (start 100 126.5) (end 100 104.13) (width 0.2) (layer "F.Cu") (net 3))
 (segment (start 109.6 136.1) (end 109.6 143) (width 0.2) (layer "F.Cu") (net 3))
 (segment (start 109.6 143) (end 111.1 144.5) (width 0.2) (layer "F.Cu") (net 3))
 (segment (start 118.699 135.801) (end 120 134.5) (width 0.2) (layer "F.Cu") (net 3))
 (segment (start 117 124.5) (end 117 138.14) (width 0.2) (layer "F.Cu") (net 2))
 (segment (start 117 138.14) (end 112.14 143) (width 0.2) (layer "F.Cu") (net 2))
 (segment (start 117.31 124.19) (end 117 124.5) (width 0.2) (layer "F.Cu") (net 2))
 (segment (start 117.31 120) (end 117.31 124.19) (width 0.2) (layer "F.Cu") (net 2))
 (segment (start 132 130) (end 138.5 130) (width 0.2) (layer "F.Cu") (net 22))
 (segment (start 138.5 130) (end 147.5 121) (width 0.2) (layer "F.Cu") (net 22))
 (segment (start 147.5 121) (end 147.5 84.32) (width 0.2) (layer "F.Cu") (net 22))
 (segment (start 147.5 84.32) (end 143.18 80) (width 0.2) (layer "F.Cu") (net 22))
 (segment (start 138.5 130) (end 139.251 129.249) (width 0.2) (layer "F.Cu") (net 22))
 (segment (start 118.931 83.929) (end 122.86 80) (width 0.2) (layer "F.Cu") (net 1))
 (segment (start 118.931 110.144) (end 118.931 83.929) (width 0.2) (layer "F.Cu") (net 1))
 (segment (start 109.075 120) (end 118.931 110.144) (width 0.2) (layer "F.Cu") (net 1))
 (segment (start 126.9 78.5) (end 125.4 80) (width 0.2) (layer "F.Cu") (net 28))
 (segment (start 135.68776 78.5) (end 126.9 78.5) (width 0.2) (layer "F.Cu") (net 28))
 (segment (start 146 110.5) (end 146 86.98776) (width 0.2) (layer "F.Cu") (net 28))
 (segment (start 126.5 130) (end 146 110.5) (width 0.2) (layer "F.Cu") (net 28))
 (segment (start 136.711 79.52324) (end 135.68776 78.5) (width 0.2) (layer "F.Cu") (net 28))
 (segment (start 146 86.98776) (end 143.222 86.98776) (width 0.2) (layer "F.Cu") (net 28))
 (segment (start 143.222 86.98776) (end 136.711 80.47676) (width 0.2) (layer "F.Cu") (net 28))
 (segment (start 136.711 80.47676) (end 136.711 79.52324) (width 0.2) (layer "F.Cu") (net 28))
 (segment (start 120 130) (end 126.5 130) (width 0.2) (layer "F.Cu") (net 28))
 (segment (start 120.07776 106) (end 121.5 104.57776) (width 0.2) (layer "F.Cu") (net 23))
 (segment (start 120 120) (end 126.5 120) (width 0.2) (layer "F.Cu") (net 23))
 (segment (start 126.5 120) (end 126.789 119.711) (width 0.2) (layer "F.Cu") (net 23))
 (segment (start 121.5 104.57776) (end 121.5 94.06) (width 0.2) (layer "F.Cu") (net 23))
 (segment (start 126.5 120) (end 126.5 115) (width 0.2) (layer "F.Cu") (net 23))
 (segment (start 120 115) (end 120 106) (width 0.2) (layer "F.Cu") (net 23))
 (segment (start 126.5 115) (end 120 115) (width 0.2) (layer "F.Cu") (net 23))
 (segment (start 121.5 94.06) (end 135.56 80) (width 0.2) (layer "F.Cu") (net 23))
 (segment (start 120 106) (end 120.07776 106) (width 0.2) (layer "F.Cu") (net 23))
 (segment (start 140.1 82) (end 138.1 80) (width 0.2) (layer "F.Cu") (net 24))
 (segment (start 146.401 86.82166) (end 141.57934 82) (width 0.2) (layer "F.Cu") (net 24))
 (segment (start 126.5 140) (end 130.5 136) (width 0.2) (layer "F.Cu") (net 24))
 (segment (start 130.5 136) (end 130.5 129.5) (width 0.2) (layer "F.Cu") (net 24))
 (segment (start 120 140) (end 126.5 140) (width 0.2) (layer "F.Cu") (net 24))
 (segment (start 146.401 113.599) (end 146.401 86.82166) (width 0.2) (layer "F.Cu") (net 24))
 (segment (start 141.57934 82) (end 140.1 82) (width 0.2) (layer "F.Cu") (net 24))
 (segment (start 130.5 129.5) (end 146.401 113.599) (width 0.2) (layer "F.Cu") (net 24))
 (segment (start 108.2115 113.02426) (end 116.629 104.60676) (width 0.2) (layer "F.Cu") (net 21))
 (segment (start 116.629 74.129) (end 134.769 74.129) (width 0.2) (layer "F.Cu") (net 21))
 (segment (start 134.769 74.129) (end 140.64 80) (width 0.2) (layer "F.Cu") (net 21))
 (segment (start 108.2115 123.7115) (end 108.2115 113.02426) (width 0.2) (layer "F.Cu") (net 21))
 (segment (start 108 130) (end 114.5 130) (width 0.2) (layer "F.Cu") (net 21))
 (segment (start 116.629 104.60676) (end 116.629 74.129) (width 0.2) (layer "F.Cu") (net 21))
 (segment (start 114.5 130) (end 108.2115 123.7115) (width 0.2) (layer "F.Cu") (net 21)))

